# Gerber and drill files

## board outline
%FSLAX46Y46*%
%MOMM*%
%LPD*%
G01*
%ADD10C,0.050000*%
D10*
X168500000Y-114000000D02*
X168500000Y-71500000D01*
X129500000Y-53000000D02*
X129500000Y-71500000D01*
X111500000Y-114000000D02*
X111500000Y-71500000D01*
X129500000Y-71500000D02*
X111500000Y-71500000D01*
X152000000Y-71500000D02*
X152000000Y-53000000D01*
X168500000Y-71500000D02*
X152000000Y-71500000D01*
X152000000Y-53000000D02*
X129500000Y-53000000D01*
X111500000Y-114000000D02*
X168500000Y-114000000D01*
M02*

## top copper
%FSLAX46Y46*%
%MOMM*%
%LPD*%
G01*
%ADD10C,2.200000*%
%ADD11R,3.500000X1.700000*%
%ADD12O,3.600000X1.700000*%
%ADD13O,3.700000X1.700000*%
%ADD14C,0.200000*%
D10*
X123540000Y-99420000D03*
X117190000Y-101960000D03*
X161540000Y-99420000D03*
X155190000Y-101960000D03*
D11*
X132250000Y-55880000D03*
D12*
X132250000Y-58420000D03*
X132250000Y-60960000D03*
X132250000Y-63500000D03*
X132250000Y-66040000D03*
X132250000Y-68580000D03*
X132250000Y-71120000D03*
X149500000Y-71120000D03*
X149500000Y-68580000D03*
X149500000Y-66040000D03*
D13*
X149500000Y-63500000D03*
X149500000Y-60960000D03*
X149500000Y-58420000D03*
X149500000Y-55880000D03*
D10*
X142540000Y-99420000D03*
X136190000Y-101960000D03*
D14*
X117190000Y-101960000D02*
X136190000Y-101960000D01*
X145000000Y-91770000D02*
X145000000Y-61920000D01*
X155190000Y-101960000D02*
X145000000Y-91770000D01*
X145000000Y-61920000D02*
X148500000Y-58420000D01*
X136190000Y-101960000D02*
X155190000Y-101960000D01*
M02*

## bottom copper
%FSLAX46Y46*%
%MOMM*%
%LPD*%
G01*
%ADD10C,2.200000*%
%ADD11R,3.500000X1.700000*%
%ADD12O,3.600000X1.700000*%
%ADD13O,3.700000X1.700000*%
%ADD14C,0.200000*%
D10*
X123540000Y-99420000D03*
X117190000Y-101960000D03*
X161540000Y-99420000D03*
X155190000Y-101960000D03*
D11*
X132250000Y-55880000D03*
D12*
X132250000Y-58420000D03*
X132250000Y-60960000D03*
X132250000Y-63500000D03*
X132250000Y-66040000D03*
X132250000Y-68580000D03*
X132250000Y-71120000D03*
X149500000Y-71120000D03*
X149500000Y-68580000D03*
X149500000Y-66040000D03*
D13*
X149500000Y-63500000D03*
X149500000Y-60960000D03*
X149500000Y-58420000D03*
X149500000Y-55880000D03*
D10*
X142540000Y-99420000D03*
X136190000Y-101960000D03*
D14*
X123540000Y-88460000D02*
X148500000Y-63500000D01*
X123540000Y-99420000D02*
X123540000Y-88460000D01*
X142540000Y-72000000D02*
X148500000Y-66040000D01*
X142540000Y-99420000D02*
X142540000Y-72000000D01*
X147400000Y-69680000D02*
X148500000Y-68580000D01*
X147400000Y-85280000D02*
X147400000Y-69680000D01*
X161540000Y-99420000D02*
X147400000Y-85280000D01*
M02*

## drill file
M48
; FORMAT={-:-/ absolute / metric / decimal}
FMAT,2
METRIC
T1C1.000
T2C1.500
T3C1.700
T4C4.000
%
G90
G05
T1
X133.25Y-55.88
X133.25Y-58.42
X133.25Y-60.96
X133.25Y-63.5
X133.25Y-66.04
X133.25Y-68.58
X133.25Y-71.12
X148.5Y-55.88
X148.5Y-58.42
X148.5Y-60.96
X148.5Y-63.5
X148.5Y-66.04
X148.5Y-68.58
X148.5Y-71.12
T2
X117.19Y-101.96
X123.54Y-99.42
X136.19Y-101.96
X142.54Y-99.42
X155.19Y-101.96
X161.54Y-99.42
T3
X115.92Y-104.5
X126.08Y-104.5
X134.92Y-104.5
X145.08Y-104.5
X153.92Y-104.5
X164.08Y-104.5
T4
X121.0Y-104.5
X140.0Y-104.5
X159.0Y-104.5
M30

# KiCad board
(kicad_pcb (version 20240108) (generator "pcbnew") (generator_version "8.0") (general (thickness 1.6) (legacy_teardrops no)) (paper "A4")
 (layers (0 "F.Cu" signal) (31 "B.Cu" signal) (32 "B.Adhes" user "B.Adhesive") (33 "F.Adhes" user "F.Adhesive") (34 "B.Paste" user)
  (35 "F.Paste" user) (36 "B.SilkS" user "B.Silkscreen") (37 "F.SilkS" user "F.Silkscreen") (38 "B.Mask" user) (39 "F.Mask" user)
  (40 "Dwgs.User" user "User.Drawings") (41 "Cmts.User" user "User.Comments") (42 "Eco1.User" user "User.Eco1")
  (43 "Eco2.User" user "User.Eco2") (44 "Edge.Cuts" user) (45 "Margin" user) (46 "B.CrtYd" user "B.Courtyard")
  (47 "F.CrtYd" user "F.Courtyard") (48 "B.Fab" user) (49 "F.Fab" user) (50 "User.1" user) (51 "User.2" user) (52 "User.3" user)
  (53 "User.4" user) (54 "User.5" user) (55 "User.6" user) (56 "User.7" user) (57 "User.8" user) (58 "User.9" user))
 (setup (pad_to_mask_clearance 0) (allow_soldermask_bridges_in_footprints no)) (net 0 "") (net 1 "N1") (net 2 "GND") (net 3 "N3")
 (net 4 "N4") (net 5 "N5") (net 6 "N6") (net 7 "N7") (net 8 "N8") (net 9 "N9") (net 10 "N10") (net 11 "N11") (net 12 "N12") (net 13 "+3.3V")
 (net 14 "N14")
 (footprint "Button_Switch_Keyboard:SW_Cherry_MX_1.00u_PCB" (layer "F.Cu") (at 123.54 99.42)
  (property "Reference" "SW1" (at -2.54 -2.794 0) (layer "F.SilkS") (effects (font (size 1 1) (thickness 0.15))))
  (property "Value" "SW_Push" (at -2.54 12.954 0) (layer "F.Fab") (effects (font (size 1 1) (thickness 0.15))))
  (pad "" np_thru_hole circle (at -7.62 5.08) (size 1.7 1.7) (drill 1.7) (layers "*.Cu" "*.Mask"))
  (pad "" np_thru_hole circle (at -2.54 5.08) (size 4 4) (drill 4) (layers "*.Cu" "*.Mask"))
  (pad "" np_thru_hole circle (at 2.54 5.08) (size 1.7 1.7) (drill 1.7) (layers "*.Cu" "*.Mask"))
  (pad "1" thru_hole circle (at 0 0) (size 2.2 2.2) (drill 1.5) (layers "*.Cu" "*.Mask") (remove_unused_layers no) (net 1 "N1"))
  (pad "2" thru_hole circle (at -6.35 2.54) (size 2.2 2.2) (drill 1.5) (layers "*.Cu" "*.Mask") (remove_unused_layers no) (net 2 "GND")))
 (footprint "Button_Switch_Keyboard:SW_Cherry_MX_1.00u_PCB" (layer "F.Cu") (at 161.54 99.42)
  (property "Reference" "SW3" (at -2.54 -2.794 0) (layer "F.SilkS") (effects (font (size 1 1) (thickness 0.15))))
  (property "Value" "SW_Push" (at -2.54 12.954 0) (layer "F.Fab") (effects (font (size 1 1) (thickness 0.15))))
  (pad "" np_thru_hole circle (at -7.62 5.08) (size 1.7 1.7) (drill 1.7) (layers "*.Cu" "*.Mask"))
  (pad "" np_thru_hole circle (at -2.54 5.08) (size 4 4) (drill 4) (layers "*.Cu" "*.Mask"))
  (pad "" np_thru_hole circle (at 2.54 5.08) (size 1.7 1.7) (drill 1.7) (layers "*.Cu" "*.Mask"))
  (pad "1" thru_hole circle (at 0 0) (size 2.2 2.2) (drill 1.5) (layers "*.Cu" "*.Mask") (remove_unused_layers no) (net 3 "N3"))
  (pad "2" thru_hole circle (at -6.35 2.54) (size 2.2 2.2) (drill 1.5) (layers "*.Cu" "*.Mask") (remove_unused_layers no) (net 2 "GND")))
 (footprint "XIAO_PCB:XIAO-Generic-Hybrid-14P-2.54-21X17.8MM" (layer "F.Cu") (at 140.875 63.5)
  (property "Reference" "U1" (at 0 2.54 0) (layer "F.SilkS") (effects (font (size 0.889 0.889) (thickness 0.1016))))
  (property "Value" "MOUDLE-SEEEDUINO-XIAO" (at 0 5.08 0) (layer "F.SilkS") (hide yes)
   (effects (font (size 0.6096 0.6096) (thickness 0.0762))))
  (pad "1" thru_hole rect (at -7.625 -7.62) (size 3.5 1.7) (drill 1 (offset -1 0)) (layers "*.Cu" "*.Mask") (remove_unused_layers no)
   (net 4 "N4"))
  (pad "2" thru_hole oval (at -7.625 -5.08) (size 3.6 1.7) (drill 1 (offset -1 0)) (layers "*.Cu" "*.Mask") (remove_unused_layers no)
   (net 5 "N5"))
  (pad "3" thru_hole oval (at -7.625 -2.54) (size 3.6 1.7) (drill 1 (offset -1 0)) (layers "*.Cu" "*.Mask") (remove_unused_layers no)
   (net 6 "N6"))
  (pad "4" thru_hole oval (at -7.625 0) (size 3.6 1.7) (drill 1 (offset -1 0)) (layers "*.Cu" "*.Mask") (remove_unused_layers no)
   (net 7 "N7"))
  (pad "5" thru_hole oval (at -7.625 2.54) (size 3.6 1.7) (drill 1 (offset -1 0)) (layers "*.Cu" "*.Mask") (remove_unused_layers no)
   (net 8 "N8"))
  (pad "6" thru_hole oval (at -7.625 5.08 180) (size 3.6 1.7) (drill 1 (offset 1 0)) (layers "*.Cu" "*.Mask") (remove_unused_layers no)
   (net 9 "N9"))
  (pad "7" thru_hole oval (at -7.625 7.62) (size 3.6 1.7) (drill 1 (offset -1 0)) (layers "*.Cu" "*.Mask") (remove_unused_layers no)
   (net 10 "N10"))
  (pad "8" thru_hole oval (at 7.625 7.62) (size 3.6 1.7) (drill 1 (offset 1 0)) (layers "*.Cu" "*.Mask") (remove_unused_layers no)
   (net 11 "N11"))
  (pad "9" thru_hole oval (at 7.625 5.08) (size 3.6 1.7) (drill 1 (offset 1 0)) (layers "*.Cu" "*.Mask") (remove_unused_layers no)
   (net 3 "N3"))
  (pad "10" thru_hole oval (at 7.625 2.54) (size 3.6 1.7) (drill 1 (offset 1 0)) (layers "*.Cu" "*.Mask") (remove_unused_layers no)
   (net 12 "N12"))
  (pad "11" thru_hole oval (at 7.625 0) (size 3.7 1.7) (drill 1 (offset 1 0)) (layers "*.Cu" "*.Mask") (remove_unused_layers no)
   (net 1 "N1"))
  (pad "12" thru_hole oval (at 7.625 -2.54) (size 3.7 1.7) (drill 1 (offset 1 0)) (layers "*.Cu" "*.Mask") (remove_unused_layers no)
   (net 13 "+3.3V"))
  (pad "13" thru_hole oval (at 7.625 -5.08) (size 3.7 1.7) (drill 1 (offset 1 0)) (layers "*.Cu" "*.Mask") (remove_unused_layers no)
   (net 2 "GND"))
  (pad "14" thru_hole oval (at 7.625 -7.62) (size 3.7 1.7) (drill 1 (offset 1 0)) (layers "*.Cu" "*.Mask") (remove_unused_layers no)
   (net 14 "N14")))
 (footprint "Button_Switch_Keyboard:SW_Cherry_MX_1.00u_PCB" (layer "F.Cu") (at 142.54 99.42)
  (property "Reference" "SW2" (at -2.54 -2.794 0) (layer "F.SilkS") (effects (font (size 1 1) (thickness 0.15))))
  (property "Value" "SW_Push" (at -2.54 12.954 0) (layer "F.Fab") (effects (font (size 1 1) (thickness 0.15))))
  (pad "" np_thru_hole circle (at -7.62 5.08) (size 1.7 1.7) (drill 1.7) (layers "*.Cu" "*.Mask"))
  (pad "" np_thru_hole circle (at -2.54 5.08) (size 4 4) (drill 4) (layers "*.Cu" "*.Mask"))
  (pad "" np_thru_hole circle (at 2.54 5.08) (size 1.7 1.7) (drill 1.7) (layers "*.Cu" "*.Mask"))
  (pad "1" thru_hole circle (at 0 0) (size 2.2 2.2) (drill 1.5) (layers "*.Cu" "*.Mask") (remove_unused_layers no) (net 12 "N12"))
  (pad "2" thru_hole circle (at -6.35 2.54) (size 2.2 2.2) (drill 1.5) (layers "*.Cu" "*.Mask") (remove_unused_layers no) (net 2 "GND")))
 (gr_line (start 168.5 114) (end 168.5 71.5) (stroke (width 0.05) (type default)) (layer "Edge.Cuts"))
 (gr_line (start 129.5 53) (end 129.5 71.5) (stroke (width 0.05) (type default)) (layer "Edge.Cuts"))
 (gr_line (start 111.5 114) (end 111.5 71.5) (stroke (width 0.05) (type default)) (layer "Edge.Cuts"))
 (gr_line (start 129.5 71.5) (end 111.5 71.5) (stroke (width 0.05) (type default)) (layer "Edge.Cuts"))
 (gr_line (start 152 71.5) (end 152 53) (stroke (width 0.05) (type default)) (layer "Edge.Cuts"))
 (gr_line (start 168.5 71.5) (end 152 71.5) (stroke (width 0.05) (type default)) (layer "Edge.Cuts"))
 (gr_line (start 152 53) (end 129.5 53) (stroke (width 0.05) (type default)) (layer "Edge.Cuts"))
 (gr_line (start 111.5 114) (end 168.5 114) (stroke (width 0.05) (type default)) (layer "Edge.Cuts"))
 (segment (start 123.54 88.46) (end 148.5 63.5) (width 0.2) (layer "B.Cu") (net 1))
 (segment (start 123.54 99.42) (end 123.54 88.46) (width 0.2) (layer "B.Cu") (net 1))
 (segment (start 142.54 72) (end 148.5 66.04) (width 0.2) (layer "B.Cu") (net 12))
 (segment (start 142.54 99.42) (end 142.54 72) (width 0.2) (layer "B.Cu") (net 12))
 (segment (start 147.4 69.68) (end 148.5 68.58) (width 0.2) (layer "B.Cu") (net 3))
 (segment (start 147.4 85.28) (end 147.4 69.68) (width 0.2) (layer "B.Cu") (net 3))
 (segment (start 161.54 99.42) (end 147.4 85.28) (width 0.2) (layer "B.Cu") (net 3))
 (segment (start 117.19 101.96) (end 136.19 101.96) (width 0.2) (layer "F.Cu") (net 2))
 (segment (start 145 91.77) (end 145 61.92) (width 0.2) (layer "F.Cu") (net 2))
 (segment (start 155.19 101.96) (end 145 91.77) (width 0.2) (layer "F.Cu") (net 2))
 (segment (start 145 61.92) (end 148.5 58.42) (width 0.2) (layer "F.Cu") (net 2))
 (segment (start 136.19 101.96) (end 155.19 101.96) (width 0.2) (layer "F.Cu") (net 2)))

